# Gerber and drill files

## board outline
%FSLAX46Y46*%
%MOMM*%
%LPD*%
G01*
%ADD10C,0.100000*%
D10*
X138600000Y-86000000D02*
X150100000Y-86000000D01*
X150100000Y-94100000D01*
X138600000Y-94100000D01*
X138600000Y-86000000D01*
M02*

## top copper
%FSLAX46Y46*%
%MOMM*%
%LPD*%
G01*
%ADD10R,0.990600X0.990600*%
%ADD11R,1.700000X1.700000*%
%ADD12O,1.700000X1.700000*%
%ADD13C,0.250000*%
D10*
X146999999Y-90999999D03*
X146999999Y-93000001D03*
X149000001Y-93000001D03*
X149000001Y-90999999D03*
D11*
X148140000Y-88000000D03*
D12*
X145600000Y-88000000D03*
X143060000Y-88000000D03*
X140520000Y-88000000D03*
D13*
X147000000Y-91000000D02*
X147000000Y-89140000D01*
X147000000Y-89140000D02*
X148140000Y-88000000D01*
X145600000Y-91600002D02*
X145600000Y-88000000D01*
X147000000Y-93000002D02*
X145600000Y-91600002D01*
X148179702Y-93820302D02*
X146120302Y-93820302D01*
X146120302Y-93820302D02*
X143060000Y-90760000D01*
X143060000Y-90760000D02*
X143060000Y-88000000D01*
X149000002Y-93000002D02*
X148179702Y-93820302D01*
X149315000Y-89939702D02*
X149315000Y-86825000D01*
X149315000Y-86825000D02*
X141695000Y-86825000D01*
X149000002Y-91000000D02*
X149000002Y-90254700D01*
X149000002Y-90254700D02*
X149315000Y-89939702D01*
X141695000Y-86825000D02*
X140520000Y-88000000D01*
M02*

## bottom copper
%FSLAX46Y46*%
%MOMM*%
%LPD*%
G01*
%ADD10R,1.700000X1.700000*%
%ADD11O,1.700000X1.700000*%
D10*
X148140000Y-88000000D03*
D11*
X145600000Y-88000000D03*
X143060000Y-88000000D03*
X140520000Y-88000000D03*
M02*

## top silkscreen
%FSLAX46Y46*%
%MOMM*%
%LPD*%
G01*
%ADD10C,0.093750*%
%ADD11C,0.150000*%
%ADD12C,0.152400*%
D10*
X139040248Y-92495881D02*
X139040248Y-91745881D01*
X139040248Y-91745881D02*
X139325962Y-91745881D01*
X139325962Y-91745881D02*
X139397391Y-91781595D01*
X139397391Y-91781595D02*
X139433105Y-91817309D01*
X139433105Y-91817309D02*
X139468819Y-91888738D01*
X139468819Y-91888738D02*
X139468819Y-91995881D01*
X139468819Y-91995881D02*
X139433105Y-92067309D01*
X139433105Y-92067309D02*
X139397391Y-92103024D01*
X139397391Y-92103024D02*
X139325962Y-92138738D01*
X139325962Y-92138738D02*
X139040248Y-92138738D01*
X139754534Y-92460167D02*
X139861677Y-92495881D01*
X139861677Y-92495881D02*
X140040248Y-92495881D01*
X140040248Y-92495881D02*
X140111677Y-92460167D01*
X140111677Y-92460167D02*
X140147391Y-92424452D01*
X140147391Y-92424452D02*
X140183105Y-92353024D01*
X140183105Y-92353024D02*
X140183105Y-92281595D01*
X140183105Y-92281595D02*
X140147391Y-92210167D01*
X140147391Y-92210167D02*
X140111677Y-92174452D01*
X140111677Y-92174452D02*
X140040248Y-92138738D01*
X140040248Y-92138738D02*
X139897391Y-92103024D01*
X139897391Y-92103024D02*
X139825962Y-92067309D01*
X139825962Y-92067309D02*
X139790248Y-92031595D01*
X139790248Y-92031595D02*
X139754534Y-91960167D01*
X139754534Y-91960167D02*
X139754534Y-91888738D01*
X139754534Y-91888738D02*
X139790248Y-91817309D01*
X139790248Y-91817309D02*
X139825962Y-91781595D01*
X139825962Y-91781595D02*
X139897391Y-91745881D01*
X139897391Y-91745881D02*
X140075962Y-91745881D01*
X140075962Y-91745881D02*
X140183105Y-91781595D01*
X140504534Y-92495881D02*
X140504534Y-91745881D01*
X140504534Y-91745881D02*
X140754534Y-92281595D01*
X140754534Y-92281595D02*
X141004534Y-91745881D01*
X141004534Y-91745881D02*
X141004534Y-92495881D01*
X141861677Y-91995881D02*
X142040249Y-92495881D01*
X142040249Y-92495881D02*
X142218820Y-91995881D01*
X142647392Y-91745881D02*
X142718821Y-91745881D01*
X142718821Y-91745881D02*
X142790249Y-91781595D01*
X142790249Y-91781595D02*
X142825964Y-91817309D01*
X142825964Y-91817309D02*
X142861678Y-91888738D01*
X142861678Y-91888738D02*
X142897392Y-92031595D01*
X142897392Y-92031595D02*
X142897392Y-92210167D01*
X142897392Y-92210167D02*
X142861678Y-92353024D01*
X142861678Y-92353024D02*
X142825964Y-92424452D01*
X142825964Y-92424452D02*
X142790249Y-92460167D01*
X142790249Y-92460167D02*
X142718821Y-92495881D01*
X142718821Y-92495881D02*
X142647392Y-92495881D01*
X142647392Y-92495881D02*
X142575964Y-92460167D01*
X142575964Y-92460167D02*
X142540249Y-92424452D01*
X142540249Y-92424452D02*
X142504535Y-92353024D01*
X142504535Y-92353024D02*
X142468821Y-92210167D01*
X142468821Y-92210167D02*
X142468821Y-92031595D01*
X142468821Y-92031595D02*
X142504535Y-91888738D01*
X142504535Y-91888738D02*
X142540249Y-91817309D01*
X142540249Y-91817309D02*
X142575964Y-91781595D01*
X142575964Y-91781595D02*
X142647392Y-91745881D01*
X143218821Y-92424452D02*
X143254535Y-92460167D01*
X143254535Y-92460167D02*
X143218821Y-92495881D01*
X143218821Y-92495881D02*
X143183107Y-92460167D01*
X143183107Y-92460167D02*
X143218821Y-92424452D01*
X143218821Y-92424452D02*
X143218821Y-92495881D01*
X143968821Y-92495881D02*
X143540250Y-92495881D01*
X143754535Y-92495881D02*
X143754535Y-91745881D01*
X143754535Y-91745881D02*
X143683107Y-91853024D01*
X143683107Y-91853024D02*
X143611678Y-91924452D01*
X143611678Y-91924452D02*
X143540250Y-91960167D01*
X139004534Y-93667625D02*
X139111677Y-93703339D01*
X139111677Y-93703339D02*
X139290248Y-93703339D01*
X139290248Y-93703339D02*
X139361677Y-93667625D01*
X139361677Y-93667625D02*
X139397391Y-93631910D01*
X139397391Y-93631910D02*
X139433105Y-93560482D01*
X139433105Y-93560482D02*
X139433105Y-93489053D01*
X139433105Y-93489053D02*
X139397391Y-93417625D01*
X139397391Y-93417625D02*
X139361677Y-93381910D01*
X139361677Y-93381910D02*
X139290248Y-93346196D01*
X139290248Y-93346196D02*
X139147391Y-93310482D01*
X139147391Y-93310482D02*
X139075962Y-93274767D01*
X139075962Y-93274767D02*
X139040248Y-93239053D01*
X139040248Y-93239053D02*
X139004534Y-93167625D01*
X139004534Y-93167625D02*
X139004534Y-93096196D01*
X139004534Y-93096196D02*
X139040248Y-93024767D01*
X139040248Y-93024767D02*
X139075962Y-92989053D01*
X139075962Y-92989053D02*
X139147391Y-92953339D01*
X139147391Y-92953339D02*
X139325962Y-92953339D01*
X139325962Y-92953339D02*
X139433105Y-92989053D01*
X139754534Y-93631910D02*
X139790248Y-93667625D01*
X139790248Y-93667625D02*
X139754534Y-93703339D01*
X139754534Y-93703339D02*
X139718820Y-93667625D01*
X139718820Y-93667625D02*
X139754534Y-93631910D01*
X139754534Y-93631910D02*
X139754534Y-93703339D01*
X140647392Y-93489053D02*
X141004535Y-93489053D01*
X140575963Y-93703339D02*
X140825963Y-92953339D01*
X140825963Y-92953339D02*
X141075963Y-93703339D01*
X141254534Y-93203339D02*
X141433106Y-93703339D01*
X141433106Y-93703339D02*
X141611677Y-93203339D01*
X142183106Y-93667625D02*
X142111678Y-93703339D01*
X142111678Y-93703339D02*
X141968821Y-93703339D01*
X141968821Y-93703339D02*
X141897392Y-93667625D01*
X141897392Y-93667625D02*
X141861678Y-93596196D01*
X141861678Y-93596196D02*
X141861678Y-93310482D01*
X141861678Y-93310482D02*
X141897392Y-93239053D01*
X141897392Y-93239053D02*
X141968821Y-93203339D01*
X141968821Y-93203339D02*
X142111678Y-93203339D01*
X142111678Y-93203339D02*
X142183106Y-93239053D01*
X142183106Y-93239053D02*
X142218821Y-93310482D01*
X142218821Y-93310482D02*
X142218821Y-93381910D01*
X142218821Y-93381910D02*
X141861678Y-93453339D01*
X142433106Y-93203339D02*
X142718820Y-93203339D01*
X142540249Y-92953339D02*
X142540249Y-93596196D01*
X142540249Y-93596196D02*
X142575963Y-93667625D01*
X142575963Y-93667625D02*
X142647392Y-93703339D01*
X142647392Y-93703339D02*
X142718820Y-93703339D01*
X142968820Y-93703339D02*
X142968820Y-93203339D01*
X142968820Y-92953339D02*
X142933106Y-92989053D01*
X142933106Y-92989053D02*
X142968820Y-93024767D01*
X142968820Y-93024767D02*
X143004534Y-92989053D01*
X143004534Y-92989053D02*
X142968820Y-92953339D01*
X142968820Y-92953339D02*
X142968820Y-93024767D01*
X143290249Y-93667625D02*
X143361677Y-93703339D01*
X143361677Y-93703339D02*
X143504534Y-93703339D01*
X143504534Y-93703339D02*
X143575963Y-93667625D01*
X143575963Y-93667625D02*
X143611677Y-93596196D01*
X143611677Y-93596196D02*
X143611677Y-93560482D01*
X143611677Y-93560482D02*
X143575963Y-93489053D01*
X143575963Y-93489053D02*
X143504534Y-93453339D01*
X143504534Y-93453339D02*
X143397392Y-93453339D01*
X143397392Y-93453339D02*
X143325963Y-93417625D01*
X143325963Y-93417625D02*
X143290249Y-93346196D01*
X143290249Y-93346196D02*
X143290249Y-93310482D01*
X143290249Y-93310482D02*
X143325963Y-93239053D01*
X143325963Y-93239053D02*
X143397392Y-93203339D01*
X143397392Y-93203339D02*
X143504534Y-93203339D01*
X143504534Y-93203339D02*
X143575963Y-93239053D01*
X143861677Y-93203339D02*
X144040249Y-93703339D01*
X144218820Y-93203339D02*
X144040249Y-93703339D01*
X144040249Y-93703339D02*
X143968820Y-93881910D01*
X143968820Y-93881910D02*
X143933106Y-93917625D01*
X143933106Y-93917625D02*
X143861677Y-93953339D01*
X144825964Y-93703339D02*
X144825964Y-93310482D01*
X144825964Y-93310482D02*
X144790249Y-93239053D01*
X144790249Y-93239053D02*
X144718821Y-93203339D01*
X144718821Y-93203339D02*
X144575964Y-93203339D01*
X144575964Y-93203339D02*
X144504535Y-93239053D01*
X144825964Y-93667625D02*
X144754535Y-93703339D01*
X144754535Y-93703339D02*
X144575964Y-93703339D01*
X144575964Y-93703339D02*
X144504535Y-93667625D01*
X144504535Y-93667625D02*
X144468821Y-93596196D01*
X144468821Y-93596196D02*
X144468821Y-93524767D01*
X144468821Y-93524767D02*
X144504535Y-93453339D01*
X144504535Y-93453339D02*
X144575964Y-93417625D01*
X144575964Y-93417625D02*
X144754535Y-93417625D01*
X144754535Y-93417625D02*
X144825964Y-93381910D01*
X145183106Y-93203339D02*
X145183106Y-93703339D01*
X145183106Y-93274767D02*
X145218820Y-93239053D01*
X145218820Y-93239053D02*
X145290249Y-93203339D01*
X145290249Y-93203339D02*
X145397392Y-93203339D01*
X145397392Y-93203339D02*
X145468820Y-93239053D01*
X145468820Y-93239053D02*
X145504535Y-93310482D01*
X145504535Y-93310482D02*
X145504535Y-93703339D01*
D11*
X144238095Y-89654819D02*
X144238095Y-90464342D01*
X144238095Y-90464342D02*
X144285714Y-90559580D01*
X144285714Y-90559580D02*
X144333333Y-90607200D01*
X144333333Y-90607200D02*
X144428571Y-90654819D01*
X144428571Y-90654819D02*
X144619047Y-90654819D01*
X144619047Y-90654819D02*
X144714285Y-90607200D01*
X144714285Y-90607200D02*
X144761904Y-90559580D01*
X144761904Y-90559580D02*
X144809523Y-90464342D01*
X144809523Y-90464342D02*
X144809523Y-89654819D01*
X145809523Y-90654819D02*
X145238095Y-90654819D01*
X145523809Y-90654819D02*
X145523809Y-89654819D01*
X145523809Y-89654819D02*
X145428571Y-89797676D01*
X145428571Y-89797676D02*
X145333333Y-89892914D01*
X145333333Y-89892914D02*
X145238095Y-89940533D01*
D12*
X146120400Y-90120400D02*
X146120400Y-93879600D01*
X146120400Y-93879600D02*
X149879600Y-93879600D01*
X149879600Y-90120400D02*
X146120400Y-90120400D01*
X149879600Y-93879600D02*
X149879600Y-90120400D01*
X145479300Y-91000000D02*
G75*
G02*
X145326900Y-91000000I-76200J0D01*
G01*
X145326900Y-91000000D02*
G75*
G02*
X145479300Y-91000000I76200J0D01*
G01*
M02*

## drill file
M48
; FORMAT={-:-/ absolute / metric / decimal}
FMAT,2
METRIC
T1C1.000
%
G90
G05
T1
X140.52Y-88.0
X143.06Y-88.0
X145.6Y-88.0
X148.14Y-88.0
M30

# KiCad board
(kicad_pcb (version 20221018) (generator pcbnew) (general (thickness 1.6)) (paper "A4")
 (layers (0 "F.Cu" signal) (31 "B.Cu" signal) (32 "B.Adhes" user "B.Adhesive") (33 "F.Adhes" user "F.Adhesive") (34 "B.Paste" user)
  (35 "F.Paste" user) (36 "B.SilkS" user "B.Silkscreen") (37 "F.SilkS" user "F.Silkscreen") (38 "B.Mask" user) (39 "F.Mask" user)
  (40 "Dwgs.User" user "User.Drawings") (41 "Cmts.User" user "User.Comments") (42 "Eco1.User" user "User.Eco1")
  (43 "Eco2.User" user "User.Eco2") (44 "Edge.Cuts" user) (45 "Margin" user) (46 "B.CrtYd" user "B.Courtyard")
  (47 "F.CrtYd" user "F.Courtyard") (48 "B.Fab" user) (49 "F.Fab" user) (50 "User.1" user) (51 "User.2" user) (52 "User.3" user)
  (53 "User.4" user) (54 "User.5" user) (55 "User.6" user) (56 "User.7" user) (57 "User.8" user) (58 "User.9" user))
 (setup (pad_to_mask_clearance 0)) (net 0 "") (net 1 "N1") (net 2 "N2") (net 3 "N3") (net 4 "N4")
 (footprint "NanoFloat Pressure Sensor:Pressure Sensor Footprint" (layer "F.Cu") (at 148 92)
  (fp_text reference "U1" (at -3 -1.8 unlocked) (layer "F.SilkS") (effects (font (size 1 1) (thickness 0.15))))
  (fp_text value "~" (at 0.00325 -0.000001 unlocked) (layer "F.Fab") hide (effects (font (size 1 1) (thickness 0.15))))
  (fp_line (start -1.8796 -1.8796) (end -1.8796 1.8796) (stroke (width 0.1524) (type solid)) (layer "F.SilkS"))
  (fp_line (start -1.8796 1.8796) (end 1.8796 1.8796) (stroke (width 0.1524) (type solid)) (layer "F.SilkS"))
  (fp_line (start 1.8796 -1.8796) (end -1.8796 -1.8796) (stroke (width 0.1524) (type solid)) (layer "F.SilkS"))
  (fp_line (start 1.8796 1.8796) (end 1.8796 -1.8796) (stroke (width 0.1524) (type solid)) (layer "F.SilkS"))
  (fp_circle (center -2.5969 -1) (end -2.5207 -1) (stroke (width 0.1524) (type solid)) (fill none) (layer "F.SilkS"))
  (pad "1" smd rect (at -1.000001 -1.000001) (size 0.9906 0.9906) (layers "F.Cu" "F.Paste" "F.Mask") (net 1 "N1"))
  (pad "2" smd rect (at -1.000001 1.000001) (size 0.9906 0.9906) (layers "F.Cu" "F.Paste" "F.Mask") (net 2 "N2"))
  (pad "3" smd rect (at 1.000001 1.000001) (size 0.9906 0.9906) (layers "F.Cu" "F.Paste" "F.Mask") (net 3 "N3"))
  (pad "4" smd rect (at 1.000001 -1.000001) (size 0.9906 0.9906) (layers "F.Cu" "F.Paste" "F.Mask") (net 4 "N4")))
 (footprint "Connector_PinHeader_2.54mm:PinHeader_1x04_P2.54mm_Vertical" (layer "B.Cu") (at 148.14 88 90)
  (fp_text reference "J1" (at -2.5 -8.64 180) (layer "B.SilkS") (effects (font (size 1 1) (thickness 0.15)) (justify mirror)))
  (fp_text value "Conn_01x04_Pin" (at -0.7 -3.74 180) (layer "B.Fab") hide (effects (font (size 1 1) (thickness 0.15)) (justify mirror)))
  (pad "1" thru_hole rect (at 0 0 90) (size 1.7 1.7) (drill 1) (layers "*.Cu" "*.Mask") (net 1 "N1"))
  (pad "2" thru_hole oval (at 0 -2.54 90) (size 1.7 1.7) (drill 1) (layers "*.Cu" "*.Mask") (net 2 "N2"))
  (pad "3" thru_hole oval (at 0 -5.08 90) (size 1.7 1.7) (drill 1) (layers "*.Cu" "*.Mask") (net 3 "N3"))
  (pad "4" thru_hole oval (at 0 -7.62 90) (size 1.7 1.7) (drill 1) (layers "*.Cu" "*.Mask") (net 4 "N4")))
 (gr_rect (start 138.6 86) (end 150.1 94.1) (stroke (width 0.1) (type default)) (fill none) (layer "Edge.Cuts"))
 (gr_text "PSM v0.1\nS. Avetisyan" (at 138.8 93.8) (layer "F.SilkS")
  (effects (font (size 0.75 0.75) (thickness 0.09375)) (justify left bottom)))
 (segment (start 147 91) (end 147 89.14) (width 0.25) (layer "F.Cu") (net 1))
 (segment (start 147 89.14) (end 148.14 88) (width 0.25) (layer "F.Cu") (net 1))
 (segment (start 145.6 91.600002) (end 145.6 88) (width 0.25) (layer "F.Cu") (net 2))
 (segment (start 147 93.000002) (end 145.6 91.600002) (width 0.25) (layer "F.Cu") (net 2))
 (segment (start 148.179702 93.820302) (end 146.120302 93.820302) (width 0.25) (layer "F.Cu") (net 3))
 (segment (start 146.120302 93.820302) (end 143.06 90.76) (width 0.25) (layer "F.Cu") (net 3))
 (segment (start 143.06 90.76) (end 143.06 88) (width 0.25) (layer "F.Cu") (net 3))
 (segment (start 149.000002 93.000002) (end 148.179702 93.820302) (width 0.25) (layer "F.Cu") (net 3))
 (segment (start 149.315 89.939702) (end 149.315 86.825) (width 0.25) (layer "F.Cu") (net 4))
 (segment (start 149.315 86.825) (end 141.695 86.825) (width 0.25) (layer "F.Cu") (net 4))
 (segment (start 149.000002 91) (end 149.000002 90.2547) (width 0.25) (layer "F.Cu") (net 4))
 (segment (start 149.000002 90.2547) (end 149.315 89.939702) (width 0.25) (layer "F.Cu") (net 4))
 (segment (start 141.695 86.825) (end 140.52 88) (width 0.25) (layer "F.Cu") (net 4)))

